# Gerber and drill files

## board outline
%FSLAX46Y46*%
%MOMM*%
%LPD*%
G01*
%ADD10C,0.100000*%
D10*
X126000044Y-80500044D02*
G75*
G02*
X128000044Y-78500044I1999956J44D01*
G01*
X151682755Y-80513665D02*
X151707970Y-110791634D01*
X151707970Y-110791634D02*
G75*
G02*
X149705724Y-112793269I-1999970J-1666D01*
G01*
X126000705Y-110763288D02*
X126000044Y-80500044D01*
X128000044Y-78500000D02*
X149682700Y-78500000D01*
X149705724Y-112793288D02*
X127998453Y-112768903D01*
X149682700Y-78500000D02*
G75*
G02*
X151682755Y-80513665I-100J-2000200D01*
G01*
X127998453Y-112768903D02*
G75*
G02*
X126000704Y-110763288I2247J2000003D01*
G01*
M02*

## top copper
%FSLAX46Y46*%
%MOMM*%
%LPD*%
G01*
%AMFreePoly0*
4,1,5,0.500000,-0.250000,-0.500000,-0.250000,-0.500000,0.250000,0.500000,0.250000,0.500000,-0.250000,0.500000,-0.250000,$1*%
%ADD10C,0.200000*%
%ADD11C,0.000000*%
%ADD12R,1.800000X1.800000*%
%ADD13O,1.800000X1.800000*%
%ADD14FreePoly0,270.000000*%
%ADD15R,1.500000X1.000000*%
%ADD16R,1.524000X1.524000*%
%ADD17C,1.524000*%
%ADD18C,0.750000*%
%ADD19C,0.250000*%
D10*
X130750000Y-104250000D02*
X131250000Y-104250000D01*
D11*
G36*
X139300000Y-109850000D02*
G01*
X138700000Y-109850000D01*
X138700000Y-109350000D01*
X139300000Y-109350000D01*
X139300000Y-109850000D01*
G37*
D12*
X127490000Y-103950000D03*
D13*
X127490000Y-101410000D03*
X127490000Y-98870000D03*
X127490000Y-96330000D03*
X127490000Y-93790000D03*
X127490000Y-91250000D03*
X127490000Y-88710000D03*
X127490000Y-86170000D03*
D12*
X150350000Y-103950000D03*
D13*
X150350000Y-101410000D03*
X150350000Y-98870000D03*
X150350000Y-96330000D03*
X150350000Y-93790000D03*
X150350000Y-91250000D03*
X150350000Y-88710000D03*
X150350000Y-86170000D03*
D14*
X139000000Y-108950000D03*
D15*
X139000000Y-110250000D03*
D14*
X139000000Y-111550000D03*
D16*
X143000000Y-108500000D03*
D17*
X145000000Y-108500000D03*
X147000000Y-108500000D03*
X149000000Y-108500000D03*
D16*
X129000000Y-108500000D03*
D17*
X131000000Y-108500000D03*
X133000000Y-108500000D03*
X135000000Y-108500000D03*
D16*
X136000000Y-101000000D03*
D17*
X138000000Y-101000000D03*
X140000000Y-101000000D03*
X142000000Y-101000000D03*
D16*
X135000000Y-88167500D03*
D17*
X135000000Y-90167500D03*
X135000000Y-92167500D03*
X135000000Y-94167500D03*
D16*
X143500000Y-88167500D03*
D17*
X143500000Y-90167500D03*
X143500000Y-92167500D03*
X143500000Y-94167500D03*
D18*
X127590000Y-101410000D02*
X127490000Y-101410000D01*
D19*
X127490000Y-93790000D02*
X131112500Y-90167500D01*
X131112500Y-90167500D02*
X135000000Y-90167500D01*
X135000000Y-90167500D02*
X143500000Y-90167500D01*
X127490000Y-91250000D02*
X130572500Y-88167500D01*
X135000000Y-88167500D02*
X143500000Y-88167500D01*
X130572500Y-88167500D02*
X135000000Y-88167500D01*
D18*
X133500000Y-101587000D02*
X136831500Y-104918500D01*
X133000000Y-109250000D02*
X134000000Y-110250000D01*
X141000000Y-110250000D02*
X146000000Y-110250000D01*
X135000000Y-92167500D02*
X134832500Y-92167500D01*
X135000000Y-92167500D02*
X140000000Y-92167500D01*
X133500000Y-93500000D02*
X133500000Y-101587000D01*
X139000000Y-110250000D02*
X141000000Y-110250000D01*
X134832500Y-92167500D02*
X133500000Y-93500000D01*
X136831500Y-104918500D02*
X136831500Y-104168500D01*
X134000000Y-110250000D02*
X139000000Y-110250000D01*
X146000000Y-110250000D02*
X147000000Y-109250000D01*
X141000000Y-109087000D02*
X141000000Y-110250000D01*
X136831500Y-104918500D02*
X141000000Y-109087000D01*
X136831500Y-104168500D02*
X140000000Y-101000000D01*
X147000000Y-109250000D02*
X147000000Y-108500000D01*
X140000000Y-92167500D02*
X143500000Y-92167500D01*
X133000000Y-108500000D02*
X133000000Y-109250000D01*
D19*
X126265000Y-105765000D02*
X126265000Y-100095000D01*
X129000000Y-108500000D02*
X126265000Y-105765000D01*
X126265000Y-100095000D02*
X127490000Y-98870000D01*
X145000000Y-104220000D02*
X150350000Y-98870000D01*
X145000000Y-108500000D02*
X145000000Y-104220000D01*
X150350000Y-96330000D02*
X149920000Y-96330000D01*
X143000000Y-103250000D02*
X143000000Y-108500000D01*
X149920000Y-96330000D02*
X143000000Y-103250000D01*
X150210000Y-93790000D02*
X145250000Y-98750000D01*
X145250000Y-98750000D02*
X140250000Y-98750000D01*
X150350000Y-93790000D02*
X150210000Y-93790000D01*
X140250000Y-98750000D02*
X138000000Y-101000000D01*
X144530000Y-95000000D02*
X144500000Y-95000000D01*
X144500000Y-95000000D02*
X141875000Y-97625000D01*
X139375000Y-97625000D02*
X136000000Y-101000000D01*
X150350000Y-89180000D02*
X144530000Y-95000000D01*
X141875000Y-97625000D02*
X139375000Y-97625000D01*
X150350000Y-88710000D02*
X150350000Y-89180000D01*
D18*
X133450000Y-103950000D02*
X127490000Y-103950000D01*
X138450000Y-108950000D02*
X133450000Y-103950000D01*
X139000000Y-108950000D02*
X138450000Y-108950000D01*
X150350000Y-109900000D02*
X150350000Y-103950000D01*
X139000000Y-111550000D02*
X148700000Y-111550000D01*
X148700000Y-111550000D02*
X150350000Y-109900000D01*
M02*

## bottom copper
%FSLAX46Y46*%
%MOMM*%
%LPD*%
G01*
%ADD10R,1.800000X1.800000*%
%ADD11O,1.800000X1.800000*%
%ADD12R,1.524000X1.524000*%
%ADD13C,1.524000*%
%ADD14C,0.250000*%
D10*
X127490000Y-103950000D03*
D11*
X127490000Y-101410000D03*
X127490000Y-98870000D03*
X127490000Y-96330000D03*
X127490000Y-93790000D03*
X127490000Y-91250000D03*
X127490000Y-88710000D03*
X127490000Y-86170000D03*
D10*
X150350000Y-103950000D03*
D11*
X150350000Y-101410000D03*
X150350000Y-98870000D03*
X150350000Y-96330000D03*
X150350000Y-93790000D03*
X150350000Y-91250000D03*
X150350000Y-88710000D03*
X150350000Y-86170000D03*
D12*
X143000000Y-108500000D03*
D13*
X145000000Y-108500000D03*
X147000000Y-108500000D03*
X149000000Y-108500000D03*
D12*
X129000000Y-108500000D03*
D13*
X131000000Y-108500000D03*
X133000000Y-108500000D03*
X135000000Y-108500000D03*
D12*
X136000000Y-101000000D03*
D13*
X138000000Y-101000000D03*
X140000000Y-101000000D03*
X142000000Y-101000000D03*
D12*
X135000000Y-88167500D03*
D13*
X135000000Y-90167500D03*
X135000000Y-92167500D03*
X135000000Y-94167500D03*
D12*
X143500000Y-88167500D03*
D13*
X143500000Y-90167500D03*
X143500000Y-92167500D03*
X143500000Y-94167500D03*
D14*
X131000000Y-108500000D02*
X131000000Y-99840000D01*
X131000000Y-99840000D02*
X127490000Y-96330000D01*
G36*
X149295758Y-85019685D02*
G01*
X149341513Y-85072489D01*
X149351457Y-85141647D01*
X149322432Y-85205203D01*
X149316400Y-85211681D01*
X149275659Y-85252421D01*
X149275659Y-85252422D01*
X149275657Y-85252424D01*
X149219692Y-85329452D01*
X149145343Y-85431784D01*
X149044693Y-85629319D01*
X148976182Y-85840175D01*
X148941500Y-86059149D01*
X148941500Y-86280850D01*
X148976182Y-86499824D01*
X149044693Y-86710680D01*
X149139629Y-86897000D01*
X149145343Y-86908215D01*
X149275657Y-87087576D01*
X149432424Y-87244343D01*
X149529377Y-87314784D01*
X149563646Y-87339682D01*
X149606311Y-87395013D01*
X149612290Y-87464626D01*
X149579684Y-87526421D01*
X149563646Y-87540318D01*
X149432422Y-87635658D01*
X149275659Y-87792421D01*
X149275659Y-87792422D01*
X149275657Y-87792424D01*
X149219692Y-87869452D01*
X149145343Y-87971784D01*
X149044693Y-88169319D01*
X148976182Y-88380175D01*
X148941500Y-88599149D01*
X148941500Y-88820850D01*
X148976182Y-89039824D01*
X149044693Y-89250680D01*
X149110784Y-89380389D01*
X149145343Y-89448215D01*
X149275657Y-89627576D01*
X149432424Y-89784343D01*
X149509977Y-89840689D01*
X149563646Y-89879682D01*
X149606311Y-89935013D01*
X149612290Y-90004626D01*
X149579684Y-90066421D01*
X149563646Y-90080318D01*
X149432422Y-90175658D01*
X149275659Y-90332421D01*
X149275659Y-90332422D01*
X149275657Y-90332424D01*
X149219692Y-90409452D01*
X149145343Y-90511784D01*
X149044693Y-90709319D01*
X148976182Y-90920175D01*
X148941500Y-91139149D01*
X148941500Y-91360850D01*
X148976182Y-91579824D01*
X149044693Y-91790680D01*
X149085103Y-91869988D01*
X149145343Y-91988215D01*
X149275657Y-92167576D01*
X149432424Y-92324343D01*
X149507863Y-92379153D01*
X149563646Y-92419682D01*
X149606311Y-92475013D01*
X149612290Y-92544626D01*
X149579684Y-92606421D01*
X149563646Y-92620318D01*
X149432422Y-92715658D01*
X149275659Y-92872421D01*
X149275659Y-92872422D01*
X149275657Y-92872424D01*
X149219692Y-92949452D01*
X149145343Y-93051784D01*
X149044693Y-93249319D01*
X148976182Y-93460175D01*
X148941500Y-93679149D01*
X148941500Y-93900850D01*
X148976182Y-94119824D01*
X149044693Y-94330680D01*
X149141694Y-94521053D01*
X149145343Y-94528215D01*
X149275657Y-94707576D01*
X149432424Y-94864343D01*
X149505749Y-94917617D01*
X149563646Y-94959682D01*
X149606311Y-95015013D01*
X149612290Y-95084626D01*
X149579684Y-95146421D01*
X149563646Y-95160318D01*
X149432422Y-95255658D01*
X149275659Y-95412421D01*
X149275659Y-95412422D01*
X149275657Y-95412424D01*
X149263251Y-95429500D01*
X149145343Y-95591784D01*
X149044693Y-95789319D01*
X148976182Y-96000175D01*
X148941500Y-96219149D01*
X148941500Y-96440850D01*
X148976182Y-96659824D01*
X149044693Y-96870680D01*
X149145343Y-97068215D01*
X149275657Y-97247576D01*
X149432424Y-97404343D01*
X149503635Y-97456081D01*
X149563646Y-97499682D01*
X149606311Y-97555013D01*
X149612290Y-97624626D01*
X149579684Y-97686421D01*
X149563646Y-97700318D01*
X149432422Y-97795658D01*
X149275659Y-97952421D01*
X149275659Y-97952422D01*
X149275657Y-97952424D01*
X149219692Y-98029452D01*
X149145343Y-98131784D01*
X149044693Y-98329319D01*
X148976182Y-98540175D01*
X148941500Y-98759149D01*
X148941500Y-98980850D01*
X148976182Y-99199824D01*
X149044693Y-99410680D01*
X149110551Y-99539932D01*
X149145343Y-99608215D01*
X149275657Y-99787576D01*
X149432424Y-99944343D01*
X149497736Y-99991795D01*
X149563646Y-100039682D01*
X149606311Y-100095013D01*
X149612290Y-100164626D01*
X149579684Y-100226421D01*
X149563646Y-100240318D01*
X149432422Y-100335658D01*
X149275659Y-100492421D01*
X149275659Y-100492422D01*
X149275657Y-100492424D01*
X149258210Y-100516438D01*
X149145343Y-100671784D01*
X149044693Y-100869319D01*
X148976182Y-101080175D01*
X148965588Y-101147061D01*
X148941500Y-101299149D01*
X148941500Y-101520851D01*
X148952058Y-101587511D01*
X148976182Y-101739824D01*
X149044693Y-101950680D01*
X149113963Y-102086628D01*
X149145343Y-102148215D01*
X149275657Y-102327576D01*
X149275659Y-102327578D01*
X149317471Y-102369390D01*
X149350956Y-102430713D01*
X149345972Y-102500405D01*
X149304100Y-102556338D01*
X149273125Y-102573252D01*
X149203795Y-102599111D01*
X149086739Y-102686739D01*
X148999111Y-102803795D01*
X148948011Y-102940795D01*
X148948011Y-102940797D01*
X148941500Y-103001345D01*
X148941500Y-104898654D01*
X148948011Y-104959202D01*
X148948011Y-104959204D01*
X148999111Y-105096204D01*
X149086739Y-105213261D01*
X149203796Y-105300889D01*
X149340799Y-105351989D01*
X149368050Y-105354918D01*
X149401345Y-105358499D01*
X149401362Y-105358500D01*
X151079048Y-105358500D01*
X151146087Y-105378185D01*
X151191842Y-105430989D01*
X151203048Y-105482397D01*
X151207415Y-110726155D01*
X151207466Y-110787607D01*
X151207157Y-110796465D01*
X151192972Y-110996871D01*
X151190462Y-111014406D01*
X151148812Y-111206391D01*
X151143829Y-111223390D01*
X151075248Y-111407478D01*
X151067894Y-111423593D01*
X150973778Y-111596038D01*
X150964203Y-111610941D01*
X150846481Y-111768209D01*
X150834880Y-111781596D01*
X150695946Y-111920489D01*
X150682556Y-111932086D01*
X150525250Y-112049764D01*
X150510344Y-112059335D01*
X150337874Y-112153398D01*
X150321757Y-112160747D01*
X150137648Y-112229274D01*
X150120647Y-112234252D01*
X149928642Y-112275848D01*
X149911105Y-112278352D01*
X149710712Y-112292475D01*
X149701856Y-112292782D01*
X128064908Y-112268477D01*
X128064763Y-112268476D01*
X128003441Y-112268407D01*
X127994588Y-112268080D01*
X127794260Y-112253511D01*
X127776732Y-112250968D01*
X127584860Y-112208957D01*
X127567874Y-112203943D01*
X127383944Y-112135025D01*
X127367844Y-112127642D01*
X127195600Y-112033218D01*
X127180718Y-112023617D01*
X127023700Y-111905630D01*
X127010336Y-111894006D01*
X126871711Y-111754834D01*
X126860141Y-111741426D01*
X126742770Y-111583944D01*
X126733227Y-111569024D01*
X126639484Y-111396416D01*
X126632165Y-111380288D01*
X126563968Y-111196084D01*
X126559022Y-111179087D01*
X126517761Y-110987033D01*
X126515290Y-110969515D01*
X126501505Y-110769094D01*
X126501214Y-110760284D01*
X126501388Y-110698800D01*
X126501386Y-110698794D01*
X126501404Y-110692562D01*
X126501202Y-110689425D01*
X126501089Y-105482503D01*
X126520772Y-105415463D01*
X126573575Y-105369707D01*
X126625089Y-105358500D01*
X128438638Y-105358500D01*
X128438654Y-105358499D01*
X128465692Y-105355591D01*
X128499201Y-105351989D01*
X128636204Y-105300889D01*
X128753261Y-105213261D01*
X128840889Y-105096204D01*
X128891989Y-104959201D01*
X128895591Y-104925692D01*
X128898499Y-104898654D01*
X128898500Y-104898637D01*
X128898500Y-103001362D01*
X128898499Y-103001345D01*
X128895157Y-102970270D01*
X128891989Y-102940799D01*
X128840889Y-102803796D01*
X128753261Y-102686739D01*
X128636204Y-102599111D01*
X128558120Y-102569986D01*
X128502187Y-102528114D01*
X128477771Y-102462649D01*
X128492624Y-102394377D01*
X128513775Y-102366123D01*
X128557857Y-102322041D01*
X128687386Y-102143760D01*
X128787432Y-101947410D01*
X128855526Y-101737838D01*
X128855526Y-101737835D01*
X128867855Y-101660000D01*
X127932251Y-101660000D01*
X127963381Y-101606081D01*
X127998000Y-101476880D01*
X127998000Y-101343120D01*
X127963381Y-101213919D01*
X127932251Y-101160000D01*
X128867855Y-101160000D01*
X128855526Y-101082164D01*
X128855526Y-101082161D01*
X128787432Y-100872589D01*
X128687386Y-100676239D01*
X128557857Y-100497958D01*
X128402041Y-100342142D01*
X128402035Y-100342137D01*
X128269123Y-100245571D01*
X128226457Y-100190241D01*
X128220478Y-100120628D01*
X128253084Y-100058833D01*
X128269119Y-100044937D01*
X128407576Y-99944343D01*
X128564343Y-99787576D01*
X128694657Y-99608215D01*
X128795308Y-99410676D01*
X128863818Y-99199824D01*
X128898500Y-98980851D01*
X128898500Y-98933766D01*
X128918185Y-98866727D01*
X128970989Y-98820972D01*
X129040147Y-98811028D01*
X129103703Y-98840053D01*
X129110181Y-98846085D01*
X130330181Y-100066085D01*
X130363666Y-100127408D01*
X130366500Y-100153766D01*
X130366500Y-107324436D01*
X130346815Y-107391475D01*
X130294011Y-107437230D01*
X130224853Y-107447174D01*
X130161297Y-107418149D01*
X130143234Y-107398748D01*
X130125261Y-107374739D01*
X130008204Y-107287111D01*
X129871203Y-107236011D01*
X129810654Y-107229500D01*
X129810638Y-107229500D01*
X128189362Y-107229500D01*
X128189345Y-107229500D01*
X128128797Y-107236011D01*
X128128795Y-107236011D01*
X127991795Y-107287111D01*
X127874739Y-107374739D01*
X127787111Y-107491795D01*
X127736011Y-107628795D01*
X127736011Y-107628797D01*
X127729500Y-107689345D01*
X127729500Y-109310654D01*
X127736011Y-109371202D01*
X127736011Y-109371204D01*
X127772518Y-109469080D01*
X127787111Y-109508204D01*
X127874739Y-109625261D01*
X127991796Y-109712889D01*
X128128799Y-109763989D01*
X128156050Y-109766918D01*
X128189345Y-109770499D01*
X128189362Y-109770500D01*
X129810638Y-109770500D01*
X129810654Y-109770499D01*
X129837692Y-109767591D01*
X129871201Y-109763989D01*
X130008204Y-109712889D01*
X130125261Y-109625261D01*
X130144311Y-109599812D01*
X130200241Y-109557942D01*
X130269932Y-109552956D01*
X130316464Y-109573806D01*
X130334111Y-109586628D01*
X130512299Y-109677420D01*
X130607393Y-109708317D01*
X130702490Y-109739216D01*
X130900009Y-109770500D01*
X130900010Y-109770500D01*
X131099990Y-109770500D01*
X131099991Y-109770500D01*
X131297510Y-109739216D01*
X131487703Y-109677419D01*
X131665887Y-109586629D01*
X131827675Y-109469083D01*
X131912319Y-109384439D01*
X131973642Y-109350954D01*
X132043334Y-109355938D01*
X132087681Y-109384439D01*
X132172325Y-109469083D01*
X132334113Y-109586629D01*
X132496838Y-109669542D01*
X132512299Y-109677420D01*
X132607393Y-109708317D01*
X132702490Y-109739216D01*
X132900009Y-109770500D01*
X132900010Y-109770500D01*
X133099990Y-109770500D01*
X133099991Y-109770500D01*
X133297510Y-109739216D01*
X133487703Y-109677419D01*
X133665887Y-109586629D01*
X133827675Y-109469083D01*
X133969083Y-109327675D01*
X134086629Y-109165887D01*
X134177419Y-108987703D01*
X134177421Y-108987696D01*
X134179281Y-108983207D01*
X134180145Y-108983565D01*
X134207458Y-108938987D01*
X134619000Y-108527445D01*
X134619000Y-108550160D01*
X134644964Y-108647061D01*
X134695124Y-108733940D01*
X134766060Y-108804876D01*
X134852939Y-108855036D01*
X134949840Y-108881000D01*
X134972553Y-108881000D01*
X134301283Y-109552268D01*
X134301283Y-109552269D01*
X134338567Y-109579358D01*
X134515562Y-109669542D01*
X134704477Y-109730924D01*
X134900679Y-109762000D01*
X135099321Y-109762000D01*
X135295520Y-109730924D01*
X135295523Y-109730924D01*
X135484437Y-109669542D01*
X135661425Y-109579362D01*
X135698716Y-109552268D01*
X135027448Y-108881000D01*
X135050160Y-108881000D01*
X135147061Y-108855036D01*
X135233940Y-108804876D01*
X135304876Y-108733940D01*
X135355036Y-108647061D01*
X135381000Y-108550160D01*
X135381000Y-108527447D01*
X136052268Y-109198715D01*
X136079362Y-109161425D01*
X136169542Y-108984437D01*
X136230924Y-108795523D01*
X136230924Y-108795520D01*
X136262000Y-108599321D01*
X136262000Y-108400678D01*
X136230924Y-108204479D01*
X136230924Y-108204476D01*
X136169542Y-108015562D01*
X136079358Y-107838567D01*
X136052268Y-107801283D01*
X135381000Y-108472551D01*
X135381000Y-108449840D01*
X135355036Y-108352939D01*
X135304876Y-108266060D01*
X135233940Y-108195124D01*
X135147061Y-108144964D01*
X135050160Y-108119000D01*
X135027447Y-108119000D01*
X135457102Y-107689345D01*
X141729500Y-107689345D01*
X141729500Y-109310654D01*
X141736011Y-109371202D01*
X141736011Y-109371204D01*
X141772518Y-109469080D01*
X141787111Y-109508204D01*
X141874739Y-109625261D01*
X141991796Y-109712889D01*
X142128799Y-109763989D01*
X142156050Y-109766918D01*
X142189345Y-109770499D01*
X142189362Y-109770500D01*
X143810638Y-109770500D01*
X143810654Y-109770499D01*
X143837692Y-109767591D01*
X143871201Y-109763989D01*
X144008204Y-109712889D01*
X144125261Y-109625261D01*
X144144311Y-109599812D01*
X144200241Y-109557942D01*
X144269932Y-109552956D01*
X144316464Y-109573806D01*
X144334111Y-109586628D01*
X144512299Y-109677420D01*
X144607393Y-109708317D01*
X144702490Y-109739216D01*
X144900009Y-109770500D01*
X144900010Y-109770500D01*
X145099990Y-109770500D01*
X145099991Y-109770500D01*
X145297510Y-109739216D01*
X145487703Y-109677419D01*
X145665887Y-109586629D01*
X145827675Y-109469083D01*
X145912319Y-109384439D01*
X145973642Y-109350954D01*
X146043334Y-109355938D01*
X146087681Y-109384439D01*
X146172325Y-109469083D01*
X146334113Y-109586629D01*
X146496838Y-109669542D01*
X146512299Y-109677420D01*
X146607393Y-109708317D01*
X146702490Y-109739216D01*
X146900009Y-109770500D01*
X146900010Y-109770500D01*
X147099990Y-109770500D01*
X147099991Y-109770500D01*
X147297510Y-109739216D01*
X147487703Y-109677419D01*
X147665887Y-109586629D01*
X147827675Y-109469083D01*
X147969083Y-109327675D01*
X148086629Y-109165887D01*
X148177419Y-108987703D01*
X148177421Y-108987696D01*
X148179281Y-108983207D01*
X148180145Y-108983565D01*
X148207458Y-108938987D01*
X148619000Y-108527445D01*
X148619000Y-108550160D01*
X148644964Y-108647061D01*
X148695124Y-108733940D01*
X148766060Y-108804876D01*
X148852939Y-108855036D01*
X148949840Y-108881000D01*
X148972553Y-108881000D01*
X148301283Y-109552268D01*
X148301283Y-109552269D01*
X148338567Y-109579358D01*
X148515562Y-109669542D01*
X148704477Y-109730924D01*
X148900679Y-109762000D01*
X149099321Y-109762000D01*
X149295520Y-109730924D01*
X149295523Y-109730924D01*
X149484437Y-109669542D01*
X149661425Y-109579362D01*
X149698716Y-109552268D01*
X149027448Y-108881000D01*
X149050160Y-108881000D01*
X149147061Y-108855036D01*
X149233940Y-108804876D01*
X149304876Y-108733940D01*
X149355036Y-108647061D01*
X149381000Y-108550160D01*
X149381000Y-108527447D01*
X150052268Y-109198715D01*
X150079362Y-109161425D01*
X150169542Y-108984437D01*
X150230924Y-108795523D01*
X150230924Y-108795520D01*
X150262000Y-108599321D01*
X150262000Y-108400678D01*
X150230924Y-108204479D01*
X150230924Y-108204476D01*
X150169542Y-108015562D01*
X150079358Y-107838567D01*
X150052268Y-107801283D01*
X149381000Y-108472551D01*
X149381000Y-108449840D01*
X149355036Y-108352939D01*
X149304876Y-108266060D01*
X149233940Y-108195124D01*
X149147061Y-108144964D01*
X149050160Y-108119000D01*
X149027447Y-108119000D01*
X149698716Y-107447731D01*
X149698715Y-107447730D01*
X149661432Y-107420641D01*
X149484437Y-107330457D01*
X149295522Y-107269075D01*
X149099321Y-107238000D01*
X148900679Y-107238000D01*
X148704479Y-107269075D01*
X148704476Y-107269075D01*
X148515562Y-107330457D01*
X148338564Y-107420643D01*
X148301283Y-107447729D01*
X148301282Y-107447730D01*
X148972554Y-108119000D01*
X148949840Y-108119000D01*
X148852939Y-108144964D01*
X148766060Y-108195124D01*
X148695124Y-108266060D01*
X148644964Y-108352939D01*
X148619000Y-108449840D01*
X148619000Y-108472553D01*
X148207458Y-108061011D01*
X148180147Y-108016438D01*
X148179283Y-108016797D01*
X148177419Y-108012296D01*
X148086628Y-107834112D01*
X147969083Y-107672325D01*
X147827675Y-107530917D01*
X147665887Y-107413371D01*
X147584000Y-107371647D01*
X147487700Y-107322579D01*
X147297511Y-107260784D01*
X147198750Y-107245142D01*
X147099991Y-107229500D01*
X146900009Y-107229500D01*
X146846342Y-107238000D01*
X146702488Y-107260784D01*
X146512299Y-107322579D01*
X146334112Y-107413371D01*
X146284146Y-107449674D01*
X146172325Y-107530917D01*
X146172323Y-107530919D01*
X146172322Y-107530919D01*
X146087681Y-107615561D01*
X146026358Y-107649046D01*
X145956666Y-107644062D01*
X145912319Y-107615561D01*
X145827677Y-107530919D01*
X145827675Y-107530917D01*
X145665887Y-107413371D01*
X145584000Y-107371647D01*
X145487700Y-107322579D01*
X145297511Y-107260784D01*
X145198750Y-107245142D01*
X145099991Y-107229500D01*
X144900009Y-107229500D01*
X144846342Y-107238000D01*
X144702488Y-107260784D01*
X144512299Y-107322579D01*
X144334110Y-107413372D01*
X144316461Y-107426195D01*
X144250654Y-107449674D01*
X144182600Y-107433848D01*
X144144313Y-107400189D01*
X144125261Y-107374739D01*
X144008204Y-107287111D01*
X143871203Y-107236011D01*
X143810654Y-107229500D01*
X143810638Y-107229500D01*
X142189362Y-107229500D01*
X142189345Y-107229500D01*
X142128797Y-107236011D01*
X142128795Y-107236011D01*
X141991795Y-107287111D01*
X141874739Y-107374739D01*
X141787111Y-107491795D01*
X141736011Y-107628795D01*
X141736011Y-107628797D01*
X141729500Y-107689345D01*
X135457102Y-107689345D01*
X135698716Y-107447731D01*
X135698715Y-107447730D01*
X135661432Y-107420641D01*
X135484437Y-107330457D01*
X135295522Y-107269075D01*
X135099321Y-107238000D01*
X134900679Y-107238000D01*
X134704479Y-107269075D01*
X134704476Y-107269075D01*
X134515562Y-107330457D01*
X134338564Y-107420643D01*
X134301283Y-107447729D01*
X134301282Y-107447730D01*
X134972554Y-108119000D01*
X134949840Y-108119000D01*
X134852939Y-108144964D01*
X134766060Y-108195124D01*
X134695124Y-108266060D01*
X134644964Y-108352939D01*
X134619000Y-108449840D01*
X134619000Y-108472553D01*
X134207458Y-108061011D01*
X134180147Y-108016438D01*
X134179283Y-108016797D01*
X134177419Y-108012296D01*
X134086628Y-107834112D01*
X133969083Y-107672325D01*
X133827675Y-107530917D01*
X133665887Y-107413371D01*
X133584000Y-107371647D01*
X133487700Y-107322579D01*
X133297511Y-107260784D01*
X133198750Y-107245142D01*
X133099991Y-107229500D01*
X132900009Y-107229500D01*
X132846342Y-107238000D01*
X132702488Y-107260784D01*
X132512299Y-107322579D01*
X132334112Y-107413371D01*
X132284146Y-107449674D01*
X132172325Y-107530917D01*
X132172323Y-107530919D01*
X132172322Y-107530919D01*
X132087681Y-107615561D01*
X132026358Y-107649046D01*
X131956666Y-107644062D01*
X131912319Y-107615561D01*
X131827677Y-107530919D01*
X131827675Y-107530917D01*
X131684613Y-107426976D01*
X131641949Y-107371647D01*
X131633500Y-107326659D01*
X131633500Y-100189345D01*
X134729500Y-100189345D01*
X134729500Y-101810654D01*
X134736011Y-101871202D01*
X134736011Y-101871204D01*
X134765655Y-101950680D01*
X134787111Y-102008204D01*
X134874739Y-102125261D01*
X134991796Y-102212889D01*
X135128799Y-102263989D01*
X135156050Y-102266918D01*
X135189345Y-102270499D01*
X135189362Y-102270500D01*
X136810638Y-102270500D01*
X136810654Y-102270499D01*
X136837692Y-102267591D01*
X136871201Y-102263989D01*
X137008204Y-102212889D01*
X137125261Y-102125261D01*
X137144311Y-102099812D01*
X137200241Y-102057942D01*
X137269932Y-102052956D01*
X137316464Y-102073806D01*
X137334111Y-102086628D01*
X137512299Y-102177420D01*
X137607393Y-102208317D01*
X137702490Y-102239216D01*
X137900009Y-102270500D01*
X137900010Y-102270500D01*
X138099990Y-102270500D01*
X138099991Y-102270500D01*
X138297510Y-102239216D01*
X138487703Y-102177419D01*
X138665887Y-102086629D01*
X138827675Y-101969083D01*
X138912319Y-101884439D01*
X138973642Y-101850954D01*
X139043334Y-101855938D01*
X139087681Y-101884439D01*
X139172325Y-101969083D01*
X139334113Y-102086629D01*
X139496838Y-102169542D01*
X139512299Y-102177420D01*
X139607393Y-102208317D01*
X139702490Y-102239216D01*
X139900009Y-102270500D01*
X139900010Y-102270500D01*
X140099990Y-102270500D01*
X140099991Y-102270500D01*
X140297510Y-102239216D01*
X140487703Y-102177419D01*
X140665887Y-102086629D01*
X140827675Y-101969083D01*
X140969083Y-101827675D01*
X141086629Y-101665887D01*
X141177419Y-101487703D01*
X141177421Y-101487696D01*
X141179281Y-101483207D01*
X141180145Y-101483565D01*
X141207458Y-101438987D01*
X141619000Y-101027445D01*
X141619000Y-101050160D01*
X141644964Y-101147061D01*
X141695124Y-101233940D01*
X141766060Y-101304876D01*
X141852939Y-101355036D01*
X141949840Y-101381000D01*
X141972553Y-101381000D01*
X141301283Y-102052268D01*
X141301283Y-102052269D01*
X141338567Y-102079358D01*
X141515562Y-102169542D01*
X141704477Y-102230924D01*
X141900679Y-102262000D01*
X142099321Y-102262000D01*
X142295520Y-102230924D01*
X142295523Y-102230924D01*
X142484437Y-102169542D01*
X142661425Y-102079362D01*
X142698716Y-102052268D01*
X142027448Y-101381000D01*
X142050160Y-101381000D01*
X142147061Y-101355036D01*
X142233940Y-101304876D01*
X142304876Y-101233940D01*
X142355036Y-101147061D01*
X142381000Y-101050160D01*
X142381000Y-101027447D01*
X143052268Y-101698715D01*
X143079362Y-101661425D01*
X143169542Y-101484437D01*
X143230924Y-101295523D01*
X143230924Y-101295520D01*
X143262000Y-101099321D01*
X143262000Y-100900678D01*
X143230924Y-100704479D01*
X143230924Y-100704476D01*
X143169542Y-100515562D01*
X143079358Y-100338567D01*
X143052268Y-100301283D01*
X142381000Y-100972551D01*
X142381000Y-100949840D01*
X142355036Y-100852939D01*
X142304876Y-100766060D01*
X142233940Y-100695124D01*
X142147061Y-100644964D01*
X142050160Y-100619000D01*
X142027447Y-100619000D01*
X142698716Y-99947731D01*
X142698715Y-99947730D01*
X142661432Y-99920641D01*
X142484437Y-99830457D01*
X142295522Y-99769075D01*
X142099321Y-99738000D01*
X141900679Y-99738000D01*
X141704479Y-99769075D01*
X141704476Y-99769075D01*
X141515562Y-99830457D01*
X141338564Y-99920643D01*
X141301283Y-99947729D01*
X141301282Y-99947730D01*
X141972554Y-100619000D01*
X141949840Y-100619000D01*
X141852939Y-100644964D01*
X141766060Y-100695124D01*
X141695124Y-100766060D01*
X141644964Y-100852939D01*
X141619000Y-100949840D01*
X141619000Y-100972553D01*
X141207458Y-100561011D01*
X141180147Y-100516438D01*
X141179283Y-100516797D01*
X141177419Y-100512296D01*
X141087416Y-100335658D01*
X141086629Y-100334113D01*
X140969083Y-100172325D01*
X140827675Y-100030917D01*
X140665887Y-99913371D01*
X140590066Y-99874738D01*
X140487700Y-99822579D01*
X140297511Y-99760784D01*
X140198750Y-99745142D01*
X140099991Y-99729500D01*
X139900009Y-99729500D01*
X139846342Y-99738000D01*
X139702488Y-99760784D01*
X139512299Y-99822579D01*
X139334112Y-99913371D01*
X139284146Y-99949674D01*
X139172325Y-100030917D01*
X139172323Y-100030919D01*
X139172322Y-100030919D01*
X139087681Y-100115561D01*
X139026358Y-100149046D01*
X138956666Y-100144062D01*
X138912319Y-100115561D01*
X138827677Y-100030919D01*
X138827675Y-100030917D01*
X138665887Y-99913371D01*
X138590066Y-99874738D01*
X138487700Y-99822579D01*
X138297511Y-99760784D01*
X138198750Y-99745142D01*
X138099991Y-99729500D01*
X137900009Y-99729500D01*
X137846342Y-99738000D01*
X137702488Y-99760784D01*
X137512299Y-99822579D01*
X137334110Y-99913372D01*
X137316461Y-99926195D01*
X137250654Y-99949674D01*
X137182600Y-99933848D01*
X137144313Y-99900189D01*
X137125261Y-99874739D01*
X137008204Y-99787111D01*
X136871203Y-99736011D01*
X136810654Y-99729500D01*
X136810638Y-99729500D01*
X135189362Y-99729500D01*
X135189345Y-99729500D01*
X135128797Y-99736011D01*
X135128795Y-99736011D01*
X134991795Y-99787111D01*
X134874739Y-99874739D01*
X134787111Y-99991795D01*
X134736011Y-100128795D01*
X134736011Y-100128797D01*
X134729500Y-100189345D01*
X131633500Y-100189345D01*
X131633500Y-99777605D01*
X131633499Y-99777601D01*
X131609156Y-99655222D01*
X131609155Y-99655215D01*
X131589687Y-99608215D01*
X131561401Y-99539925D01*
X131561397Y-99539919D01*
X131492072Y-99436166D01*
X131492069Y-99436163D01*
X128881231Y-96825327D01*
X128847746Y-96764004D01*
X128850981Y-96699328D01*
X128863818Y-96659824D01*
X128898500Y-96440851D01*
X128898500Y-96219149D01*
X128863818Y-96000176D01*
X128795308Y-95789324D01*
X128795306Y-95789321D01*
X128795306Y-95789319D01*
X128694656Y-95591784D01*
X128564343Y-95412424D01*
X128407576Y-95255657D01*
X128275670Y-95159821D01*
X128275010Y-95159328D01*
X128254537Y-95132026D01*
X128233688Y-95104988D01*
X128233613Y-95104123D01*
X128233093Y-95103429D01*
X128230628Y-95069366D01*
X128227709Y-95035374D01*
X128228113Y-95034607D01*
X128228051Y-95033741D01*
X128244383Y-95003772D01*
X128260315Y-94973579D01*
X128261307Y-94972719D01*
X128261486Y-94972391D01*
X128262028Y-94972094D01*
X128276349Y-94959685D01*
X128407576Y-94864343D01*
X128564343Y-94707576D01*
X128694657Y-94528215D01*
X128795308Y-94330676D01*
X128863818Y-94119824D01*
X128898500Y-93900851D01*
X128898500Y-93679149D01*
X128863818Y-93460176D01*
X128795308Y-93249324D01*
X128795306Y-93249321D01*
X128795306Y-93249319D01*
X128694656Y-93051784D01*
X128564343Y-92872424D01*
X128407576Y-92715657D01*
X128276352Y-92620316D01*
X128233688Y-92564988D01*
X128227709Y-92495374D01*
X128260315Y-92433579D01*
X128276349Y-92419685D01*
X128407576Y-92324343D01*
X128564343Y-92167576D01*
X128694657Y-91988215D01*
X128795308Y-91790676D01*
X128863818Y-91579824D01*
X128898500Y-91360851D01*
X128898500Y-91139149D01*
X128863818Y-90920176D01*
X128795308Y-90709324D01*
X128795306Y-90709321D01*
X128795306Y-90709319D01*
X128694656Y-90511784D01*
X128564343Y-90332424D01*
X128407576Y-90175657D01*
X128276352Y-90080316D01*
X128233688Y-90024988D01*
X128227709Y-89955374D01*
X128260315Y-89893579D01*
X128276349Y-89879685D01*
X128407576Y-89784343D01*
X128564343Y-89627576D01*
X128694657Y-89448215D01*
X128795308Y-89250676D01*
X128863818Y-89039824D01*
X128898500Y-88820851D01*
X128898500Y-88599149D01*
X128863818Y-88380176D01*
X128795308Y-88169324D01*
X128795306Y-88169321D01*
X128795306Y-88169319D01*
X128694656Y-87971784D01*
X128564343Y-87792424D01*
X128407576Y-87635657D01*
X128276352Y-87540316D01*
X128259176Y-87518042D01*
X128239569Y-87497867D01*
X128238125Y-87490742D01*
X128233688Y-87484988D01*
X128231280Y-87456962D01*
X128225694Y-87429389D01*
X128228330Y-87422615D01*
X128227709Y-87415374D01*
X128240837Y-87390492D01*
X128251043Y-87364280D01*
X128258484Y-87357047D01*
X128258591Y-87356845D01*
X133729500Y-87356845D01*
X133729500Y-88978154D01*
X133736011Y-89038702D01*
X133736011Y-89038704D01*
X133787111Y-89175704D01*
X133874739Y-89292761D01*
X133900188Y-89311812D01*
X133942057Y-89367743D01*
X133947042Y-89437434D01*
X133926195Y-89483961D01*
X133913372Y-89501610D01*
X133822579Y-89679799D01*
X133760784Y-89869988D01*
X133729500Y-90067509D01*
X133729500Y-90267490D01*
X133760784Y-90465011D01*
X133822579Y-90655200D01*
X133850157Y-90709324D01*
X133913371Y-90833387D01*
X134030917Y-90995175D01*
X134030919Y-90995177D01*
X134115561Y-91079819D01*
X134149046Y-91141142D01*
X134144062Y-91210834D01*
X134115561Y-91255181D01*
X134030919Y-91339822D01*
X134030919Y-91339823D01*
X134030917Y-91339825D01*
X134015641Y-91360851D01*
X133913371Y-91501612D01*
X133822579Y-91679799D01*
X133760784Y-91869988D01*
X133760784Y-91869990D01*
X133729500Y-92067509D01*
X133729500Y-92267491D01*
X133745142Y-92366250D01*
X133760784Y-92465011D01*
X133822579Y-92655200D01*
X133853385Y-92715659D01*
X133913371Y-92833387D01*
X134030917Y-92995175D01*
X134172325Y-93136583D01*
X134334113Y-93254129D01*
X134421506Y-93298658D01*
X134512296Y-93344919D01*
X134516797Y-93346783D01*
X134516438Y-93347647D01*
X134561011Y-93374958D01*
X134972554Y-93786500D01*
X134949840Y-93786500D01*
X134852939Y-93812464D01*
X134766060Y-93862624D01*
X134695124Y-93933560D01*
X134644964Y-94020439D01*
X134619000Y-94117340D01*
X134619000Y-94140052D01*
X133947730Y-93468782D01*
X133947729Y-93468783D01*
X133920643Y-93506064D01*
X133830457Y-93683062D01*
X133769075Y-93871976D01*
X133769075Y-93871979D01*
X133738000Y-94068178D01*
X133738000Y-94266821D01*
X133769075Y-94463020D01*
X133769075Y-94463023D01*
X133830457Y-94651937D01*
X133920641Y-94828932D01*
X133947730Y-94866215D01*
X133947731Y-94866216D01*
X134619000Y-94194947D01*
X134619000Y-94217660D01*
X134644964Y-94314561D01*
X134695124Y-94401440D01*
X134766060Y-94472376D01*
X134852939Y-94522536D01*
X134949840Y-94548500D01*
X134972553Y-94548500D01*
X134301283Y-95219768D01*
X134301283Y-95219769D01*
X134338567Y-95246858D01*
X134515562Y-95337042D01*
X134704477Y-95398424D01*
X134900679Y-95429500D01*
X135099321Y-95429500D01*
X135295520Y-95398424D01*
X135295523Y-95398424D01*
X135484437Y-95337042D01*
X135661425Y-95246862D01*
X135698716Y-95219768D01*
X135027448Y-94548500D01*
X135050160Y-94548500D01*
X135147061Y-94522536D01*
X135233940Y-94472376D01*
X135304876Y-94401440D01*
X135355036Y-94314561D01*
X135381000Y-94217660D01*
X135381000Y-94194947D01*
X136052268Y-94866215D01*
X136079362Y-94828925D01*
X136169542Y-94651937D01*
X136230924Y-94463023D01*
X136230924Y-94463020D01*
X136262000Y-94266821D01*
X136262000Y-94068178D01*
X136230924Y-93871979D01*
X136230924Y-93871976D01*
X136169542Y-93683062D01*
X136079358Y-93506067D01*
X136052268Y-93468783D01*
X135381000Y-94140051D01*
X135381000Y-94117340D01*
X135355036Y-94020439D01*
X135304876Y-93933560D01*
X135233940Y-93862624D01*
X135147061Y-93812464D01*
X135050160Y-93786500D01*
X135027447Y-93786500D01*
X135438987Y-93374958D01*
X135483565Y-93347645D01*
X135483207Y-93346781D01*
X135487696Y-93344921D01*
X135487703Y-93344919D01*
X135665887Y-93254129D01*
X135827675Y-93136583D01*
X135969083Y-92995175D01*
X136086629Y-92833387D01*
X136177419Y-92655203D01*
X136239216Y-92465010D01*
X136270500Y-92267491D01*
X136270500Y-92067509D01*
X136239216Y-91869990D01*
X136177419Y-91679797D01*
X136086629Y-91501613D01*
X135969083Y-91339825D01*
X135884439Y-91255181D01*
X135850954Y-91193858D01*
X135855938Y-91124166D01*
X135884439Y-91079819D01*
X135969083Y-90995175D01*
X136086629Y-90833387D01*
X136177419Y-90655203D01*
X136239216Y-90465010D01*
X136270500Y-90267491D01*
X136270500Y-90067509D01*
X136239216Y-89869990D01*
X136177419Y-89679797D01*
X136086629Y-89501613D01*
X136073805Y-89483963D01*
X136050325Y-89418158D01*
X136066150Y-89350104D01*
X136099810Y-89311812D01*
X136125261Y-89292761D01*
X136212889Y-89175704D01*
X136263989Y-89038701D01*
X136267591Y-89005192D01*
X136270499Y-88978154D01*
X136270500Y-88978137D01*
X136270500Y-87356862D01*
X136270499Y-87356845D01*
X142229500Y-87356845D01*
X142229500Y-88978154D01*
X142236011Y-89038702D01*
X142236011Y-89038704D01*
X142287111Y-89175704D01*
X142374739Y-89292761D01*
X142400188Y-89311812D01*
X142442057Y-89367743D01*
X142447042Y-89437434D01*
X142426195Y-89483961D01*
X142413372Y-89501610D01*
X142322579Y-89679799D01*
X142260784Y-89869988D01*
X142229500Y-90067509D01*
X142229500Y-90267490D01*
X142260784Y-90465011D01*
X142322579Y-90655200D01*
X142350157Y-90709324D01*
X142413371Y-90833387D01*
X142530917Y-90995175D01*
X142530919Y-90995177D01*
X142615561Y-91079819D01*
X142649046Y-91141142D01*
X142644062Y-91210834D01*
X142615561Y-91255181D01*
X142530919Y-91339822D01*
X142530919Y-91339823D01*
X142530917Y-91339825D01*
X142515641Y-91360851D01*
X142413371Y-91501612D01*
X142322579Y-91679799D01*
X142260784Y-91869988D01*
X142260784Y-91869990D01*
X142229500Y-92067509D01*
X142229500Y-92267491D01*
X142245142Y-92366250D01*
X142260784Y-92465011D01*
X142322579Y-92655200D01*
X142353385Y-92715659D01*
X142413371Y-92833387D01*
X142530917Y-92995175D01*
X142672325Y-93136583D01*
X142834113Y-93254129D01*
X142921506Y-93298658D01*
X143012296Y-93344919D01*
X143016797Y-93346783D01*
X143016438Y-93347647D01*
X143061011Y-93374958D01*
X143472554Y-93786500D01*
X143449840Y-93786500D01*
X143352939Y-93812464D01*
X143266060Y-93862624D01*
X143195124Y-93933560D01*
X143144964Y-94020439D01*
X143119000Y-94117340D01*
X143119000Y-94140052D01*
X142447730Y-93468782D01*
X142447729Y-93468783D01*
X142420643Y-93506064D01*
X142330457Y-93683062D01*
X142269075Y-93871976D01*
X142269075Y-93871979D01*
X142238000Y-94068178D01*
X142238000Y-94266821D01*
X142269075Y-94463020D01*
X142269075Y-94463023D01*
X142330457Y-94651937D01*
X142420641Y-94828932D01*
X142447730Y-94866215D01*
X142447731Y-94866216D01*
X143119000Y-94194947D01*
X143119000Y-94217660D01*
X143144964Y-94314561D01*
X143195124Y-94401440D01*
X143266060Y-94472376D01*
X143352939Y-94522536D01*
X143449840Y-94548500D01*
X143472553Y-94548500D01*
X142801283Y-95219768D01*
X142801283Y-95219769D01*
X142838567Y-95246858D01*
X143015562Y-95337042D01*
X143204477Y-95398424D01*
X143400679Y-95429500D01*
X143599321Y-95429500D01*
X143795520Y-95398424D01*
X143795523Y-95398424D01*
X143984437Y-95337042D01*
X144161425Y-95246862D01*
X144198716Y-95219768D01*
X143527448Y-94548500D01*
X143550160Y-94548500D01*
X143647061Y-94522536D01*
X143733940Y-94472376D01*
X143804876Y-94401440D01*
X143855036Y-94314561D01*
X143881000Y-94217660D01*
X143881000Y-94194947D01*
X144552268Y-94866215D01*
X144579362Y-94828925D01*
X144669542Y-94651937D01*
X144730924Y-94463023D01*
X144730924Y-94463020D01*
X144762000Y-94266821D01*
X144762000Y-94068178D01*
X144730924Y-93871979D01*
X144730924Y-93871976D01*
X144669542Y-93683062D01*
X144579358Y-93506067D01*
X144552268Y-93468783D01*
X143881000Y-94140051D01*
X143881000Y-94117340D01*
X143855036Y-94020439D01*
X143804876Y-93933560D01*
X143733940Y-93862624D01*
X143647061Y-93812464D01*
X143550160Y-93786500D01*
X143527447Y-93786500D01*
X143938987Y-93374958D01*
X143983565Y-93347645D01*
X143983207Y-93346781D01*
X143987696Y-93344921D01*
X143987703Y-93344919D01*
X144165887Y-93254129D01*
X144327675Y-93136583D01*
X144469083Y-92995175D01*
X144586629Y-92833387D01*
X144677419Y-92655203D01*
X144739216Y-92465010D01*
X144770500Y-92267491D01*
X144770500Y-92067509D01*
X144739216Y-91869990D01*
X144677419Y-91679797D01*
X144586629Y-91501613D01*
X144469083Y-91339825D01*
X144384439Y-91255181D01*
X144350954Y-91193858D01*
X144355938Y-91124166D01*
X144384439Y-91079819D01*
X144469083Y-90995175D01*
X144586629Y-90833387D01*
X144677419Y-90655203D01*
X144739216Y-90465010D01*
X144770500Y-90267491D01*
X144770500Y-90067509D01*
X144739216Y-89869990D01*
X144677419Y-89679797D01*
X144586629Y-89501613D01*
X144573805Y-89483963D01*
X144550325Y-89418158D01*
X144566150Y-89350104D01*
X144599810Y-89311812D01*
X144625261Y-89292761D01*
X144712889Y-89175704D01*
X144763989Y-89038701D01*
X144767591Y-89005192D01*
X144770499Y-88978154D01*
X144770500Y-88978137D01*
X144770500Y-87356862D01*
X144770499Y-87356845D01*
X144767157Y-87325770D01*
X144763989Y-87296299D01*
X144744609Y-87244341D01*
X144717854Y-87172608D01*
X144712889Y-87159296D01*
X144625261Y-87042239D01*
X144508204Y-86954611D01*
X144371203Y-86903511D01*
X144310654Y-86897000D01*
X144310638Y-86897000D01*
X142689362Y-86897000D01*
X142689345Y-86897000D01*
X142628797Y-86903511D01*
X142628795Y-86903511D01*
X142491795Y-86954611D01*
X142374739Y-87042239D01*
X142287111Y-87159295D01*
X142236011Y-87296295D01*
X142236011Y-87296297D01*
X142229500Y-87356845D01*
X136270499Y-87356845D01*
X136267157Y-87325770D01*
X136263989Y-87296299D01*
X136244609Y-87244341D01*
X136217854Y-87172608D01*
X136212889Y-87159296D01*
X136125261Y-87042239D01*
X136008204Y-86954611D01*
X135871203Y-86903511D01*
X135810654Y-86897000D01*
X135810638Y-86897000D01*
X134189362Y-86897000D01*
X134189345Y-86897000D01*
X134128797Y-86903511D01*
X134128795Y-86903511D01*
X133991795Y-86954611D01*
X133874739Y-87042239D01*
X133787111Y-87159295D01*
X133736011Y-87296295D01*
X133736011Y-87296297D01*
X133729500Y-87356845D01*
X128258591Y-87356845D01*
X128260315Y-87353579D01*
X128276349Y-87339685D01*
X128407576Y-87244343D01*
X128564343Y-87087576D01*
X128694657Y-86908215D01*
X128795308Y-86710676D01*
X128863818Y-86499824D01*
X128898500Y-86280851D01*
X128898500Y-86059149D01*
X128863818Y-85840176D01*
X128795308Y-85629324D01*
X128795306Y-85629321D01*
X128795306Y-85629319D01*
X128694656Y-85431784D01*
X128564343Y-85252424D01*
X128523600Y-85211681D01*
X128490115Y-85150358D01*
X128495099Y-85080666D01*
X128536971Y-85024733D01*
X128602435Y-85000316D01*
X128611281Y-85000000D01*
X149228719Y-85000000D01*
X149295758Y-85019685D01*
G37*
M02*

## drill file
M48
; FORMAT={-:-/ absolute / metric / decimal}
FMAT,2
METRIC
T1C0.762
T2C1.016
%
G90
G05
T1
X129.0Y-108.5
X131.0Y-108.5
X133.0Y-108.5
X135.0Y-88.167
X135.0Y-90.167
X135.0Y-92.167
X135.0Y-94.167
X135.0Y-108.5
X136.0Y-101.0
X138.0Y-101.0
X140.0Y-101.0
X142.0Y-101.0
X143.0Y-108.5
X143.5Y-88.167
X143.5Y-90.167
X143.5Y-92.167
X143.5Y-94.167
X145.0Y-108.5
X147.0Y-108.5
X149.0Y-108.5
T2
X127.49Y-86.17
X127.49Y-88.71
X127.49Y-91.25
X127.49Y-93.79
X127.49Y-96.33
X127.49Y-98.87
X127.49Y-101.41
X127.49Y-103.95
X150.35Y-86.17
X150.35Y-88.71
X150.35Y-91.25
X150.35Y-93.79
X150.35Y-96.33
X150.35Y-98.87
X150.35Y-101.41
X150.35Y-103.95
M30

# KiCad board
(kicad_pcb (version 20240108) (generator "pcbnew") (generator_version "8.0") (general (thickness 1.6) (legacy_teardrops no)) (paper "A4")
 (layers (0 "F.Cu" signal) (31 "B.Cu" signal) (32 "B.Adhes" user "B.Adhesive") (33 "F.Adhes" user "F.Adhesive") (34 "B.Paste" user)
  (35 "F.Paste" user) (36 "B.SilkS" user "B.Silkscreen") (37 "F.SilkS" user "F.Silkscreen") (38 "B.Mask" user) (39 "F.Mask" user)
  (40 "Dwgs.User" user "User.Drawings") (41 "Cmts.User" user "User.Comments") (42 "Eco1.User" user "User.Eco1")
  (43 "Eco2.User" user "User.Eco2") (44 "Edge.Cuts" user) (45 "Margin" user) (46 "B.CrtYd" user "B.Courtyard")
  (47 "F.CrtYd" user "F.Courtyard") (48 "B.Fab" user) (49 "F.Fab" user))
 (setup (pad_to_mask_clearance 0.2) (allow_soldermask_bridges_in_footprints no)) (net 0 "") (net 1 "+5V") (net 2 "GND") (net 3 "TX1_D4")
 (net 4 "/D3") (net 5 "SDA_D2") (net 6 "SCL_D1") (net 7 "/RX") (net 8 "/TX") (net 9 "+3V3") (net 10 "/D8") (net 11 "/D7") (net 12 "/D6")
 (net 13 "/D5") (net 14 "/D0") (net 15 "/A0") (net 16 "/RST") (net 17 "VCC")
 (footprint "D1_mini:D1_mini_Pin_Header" (layer "F.Cu") (at 127.49 103.95 180)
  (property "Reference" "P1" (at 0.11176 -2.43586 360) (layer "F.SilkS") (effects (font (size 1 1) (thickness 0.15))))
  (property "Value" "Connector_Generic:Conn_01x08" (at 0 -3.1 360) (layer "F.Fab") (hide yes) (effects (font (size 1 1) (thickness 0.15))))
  (pad "1" thru_hole rect (at 0 0 180) (size 1.8 1.8) (drill 1.016) (layers "*.Cu" "*.Mask" "F.SilkS") (remove_unused_layers no)
   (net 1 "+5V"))
  (pad "2" thru_hole oval (at 0 2.54 180) (size 1.8 1.8) (drill 1.016) (layers "*.Cu" "*.Mask" "F.SilkS") (remove_unused_layers no)
   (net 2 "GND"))
  (pad "3" thru_hole oval (at 0 5.08 180) (size 1.8 1.8) (drill 1.016) (layers "*.Cu" "*.Mask" "F.SilkS") (remove_unused_layers no)
   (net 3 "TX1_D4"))
  (pad "4" thru_hole oval (at 0 7.62 180) (size 1.8 1.8) (drill 1.016) (layers "*.Cu" "*.Mask" "F.SilkS") (remove_unused_layers no)
   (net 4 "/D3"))
  (pad "5" thru_hole oval (at 0 10.16 180) (size 1.8 1.8) (drill 1.016) (layers "*.Cu" "*.Mask" "F.SilkS") (remove_unused_layers no)
   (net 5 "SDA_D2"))
  (pad "6" thru_hole oval (at 0 12.7 180) (size 1.8 1.8) (drill 1.016) (layers "*.Cu" "*.Mask" "F.SilkS") (remove_unused_layers no)
   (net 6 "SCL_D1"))
  (pad "7" thru_hole oval (at 0 15.24 180) (size 1.8 1.8) (drill 1.016) (layers "*.Cu" "*.Mask" "F.SilkS") (remove_unused_layers no)
   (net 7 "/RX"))
  (pad "8" thru_hole oval (at 0 17.78 180) (size 1.8 1.8) (drill 1.016) (layers "*.Cu" "*.Mask" "F.SilkS") (remove_unused_layers no)
   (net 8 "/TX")))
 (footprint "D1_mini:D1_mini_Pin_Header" (layer "F.Cu") (at 150.35 103.95 180)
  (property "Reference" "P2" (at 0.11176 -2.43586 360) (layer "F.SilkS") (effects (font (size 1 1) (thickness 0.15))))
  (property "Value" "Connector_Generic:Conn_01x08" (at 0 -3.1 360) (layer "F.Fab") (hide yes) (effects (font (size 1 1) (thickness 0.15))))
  (pad "1" thru_hole rect (at 0 0 180) (size 1.8 1.8) (drill 1.016) (layers "*.Cu" "*.Mask" "F.SilkS") (remove_unused_layers no)
   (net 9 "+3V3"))
  (pad "2" thru_hole oval (at 0 2.54 180) (size 1.8 1.8) (drill 1.016) (layers "*.Cu" "*.Mask" "F.SilkS") (remove_unused_layers no)
   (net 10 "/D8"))
  (pad "3" thru_hole oval (at 0 5.08 180) (size 1.8 1.8) (drill 1.016) (layers "*.Cu" "*.Mask" "F.SilkS") (remove_unused_layers no)
   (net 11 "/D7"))
  (pad "4" thru_hole oval (at 0 7.62 180) (size 1.8 1.8) (drill 1.016) (layers "*.Cu" "*.Mask" "F.SilkS") (remove_unused_layers no)
   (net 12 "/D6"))
  (pad "5" thru_hole oval (at 0 10.16 180) (size 1.8 1.8) (drill 1.016) (layers "*.Cu" "*.Mask" "F.SilkS") (remove_unused_layers no)
   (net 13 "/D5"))
  (pad "6" thru_hole oval (at 0 12.7 180) (size 1.8 1.8) (drill 1.016) (layers "*.Cu" "*.Mask" "F.SilkS") (remove_unused_layers no)
   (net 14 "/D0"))
  (pad "7" thru_hole oval (at 0 15.24 180) (size 1.8 1.8) (drill 1.016) (layers "*.Cu" "*.Mask" "F.SilkS") (remove_unused_layers no)
   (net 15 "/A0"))
  (pad "8" thru_hole oval (at 0 17.78 180) (size 1.8 1.8) (drill 1.016) (layers "*.Cu" "*.Mask" "F.SilkS") (remove_unused_layers no)
   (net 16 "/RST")))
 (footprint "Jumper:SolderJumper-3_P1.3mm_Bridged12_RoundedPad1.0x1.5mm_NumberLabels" (layer "F.Cu") (at 139 110.25 -90)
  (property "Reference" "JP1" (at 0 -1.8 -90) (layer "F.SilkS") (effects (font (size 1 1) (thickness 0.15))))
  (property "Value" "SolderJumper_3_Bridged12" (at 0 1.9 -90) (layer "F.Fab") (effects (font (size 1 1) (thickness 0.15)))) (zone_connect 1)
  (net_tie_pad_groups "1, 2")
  (fp_poly (pts (xy -0.9 -0.3) (xy -0.4 -0.3) (xy -0.4 0.3) (xy -0.9 0.3)) (stroke (width 0) (type solid)) (fill solid) (layer "F.Cu"))
  (pad "1" smd custom (at -1.3 0 270) (size 1 0.5) (layers "F.Cu" "F.Mask") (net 1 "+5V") (zone_connect 2) (thermal_bridge_angle 45)
   (options (clearance outline) (anchor rect)) (primitives))
  (pad "2" smd rect (at 0 0 270) (size 1 1.5) (layers "F.Cu" "F.Mask") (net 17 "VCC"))
  (pad "3" smd custom (at 1.3 0 270) (size 1 0.5) (layers "F.Cu" "F.Mask") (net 9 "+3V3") (zone_connect 2) (thermal_bridge_angle 45)
   (options (clearance outline) (anchor rect)) (primitives)))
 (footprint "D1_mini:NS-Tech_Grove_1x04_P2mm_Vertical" (layer "B.Cu") (at 143 108.5 -90)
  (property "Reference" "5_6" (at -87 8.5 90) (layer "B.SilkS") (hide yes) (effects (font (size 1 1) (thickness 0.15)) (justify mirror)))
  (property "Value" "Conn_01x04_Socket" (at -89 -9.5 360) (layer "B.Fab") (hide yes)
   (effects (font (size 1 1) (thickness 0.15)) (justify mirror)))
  (pad "1" thru_hole rect (at 0 0 270) (size 1.524 1.524) (drill 0.762) (layers "*.Cu" "*.Mask") (remove_unused_layers no) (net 12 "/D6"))
  (pad "2" thru_hole circle (at 0 -2 270) (size 1.524 1.524) (drill 0.762) (layers "*.Cu" "*.Mask") (remove_unused_layers no) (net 11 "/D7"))
  (pad "3" thru_hole circle (at 0 -4 270) (size 1.524 1.524) (drill 0.762) (layers "*.Cu" "*.Mask") (remove_unused_layers no) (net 17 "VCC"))
  (pad "4" thru_hole circle (at 0 -6 270) (size 1.524 1.524) (drill 0.762) (layers "*.Cu" "*.Mask") (remove_unused_layers no) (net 2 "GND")))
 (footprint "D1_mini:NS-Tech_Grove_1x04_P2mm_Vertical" (layer "B.Cu") (at 129 108.5 -90)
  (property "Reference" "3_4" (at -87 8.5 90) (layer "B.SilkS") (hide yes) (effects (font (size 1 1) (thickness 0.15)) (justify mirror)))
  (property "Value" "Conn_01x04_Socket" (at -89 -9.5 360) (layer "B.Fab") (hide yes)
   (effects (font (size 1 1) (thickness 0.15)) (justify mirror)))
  (pad "1" thru_hole rect (at 0 0 270) (size 1.524 1.524) (drill 0.762) (layers "*.Cu" "*.Mask") (remove_unused_layers no) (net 3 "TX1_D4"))
  (pad "2" thru_hole circle (at 0 -2 270) (size 1.524 1.524) (drill 0.762) (layers "*.Cu" "*.Mask") (remove_unused_layers no) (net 4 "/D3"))
  (pad "3" thru_hole circle (at 0 -4 270) (size 1.524 1.524) (drill 0.762) (layers "*.Cu" "*.Mask") (remove_unused_layers no) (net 17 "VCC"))
  (pad "4" thru_hole circle (at 0 -6 270) (size 1.524 1.524) (drill 0.762) (layers "*.Cu" "*.Mask") (remove_unused_layers no) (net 2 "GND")))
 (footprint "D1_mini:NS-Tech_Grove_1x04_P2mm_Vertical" (layer "B.Cu") (at 136 101 -90)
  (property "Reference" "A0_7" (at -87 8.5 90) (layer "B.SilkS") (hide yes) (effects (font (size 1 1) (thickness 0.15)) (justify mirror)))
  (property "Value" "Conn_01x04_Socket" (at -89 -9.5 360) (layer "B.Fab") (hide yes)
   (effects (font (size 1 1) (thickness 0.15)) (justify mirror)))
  (pad "1" thru_hole rect (at 0 0 270) (size 1.524 1.524) (drill 0.762) (layers "*.Cu" "*.Mask") (remove_unused_layers no) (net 15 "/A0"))
  (pad "2" thru_hole circle (at 0 -2 270) (size 1.524 1.524) (drill 0.762) (layers "*.Cu" "*.Mask") (remove_unused_layers no) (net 13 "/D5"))
  (pad "3" thru_hole circle (at 0 -4 270) (size 1.524 1.524) (drill 0.762) (layers "*.Cu" "*.Mask") (remove_unused_layers no) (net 17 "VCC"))
  (pad "4" thru_hole circle (at 0 -6 270) (size 1.524 1.524) (drill 0.762) (layers "*.Cu" "*.Mask") (remove_unused_layers no) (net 2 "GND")))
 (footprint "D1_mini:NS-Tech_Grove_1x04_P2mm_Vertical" (layer "B.Cu") (at 135 88.1675 180)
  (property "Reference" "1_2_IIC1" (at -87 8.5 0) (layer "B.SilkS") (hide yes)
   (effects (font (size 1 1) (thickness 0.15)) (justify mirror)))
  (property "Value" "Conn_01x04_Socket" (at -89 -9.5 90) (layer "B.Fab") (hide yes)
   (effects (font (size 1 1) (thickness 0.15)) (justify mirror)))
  (pad "1" thru_hole rect (at 0 0 180) (size 1.524 1.524) (drill 0.762) (layers "*.Cu" "*.Mask") (remove_unused_layers no) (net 6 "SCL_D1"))
  (pad "2" thru_hole circle (at 0 -2 180) (size 1.524 1.524) (drill 0.762) (layers "*.Cu" "*.Mask") (remove_unused_layers no)
   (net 5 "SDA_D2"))
  (pad "3" thru_hole circle (at 0 -4 180) (size 1.524 1.524) (drill 0.762) (layers "*.Cu" "*.Mask") (remove_unused_layers no) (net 17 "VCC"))
  (pad "4" thru_hole circle (at 0 -6 180) (size 1.524 1.524) (drill 0.762) (layers "*.Cu" "*.Mask") (remove_unused_layers no) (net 2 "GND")))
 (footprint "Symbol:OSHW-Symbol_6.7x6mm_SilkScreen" (layer "B.Cu") (at 147.9 81.75 180)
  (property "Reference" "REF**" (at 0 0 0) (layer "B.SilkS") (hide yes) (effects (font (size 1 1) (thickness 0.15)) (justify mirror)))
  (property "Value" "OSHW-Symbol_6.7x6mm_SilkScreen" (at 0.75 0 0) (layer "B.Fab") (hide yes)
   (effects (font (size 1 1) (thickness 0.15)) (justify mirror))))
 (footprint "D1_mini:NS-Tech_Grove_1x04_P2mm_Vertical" (layer "B.Cu") (at 143.5 88.1675 180)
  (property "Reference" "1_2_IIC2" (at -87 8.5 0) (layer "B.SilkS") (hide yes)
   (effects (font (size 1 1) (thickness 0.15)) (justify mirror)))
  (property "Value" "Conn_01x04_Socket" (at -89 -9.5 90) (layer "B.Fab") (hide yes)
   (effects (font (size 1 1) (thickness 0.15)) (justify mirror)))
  (pad "1" thru_hole rect (at 0 0 180) (size 1.524 1.524) (drill 0.762) (layers "*.Cu" "*.Mask") (remove_unused_layers no) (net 6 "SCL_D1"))
  (pad "2" thru_hole circle (at 0 -2 180) (size 1.524 1.524) (drill 0.762) (layers "*.Cu" "*.Mask") (remove_unused_layers no)
   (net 5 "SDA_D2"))
  (pad "3" thru_hole circle (at 0 -4 180) (size 1.524 1.524) (drill 0.762) (layers "*.Cu" "*.Mask") (remove_unused_layers no) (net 17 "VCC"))
  (pad "4" thru_hole circle (at 0 -6 180) (size 1.524 1.524) (drill 0.762) (layers "*.Cu" "*.Mask") (remove_unused_layers no) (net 2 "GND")))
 (gr_line (start 130.75 104.25) (end 131.25 104.25) (stroke (width 0.2) (type default)) (layer "F.Cu") (net 1))
 (gr_arc (start 126.000044 80.500044) (mid 126.585815 79.085802) (end 128.000044 78.5) (stroke (width 0.1) (type default))
  (layer "Edge.Cuts"))
 (gr_line (start 151.682755 80.513665) (end 151.70797 110.791634) (stroke (width 0.1) (type solid)) (layer "Edge.Cuts"))
 (gr_arc (start 151.70797 110.791634) (mid 151.122062 112.207625) (end 149.705724 112.793288) (stroke (width 0.1) (type default))
  (layer "Edge.Cuts"))
 (gr_line (start 126.000705 110.763288) (end 126.000044 80.500044) (stroke (width 0.1) (type solid)) (layer "Edge.Cuts"))
 (gr_line (start 128.000044 78.5) (end 149.6827 78.5) (stroke (width 0.1) (type solid)) (layer "Edge.Cuts"))
 (gr_line (start 149.705724 112.793288) (end 127.998453 112.768903) (stroke (width 0.1) (type solid)) (layer "Edge.Cuts"))
 (gr_arc (start 149.6827 78.5) (mid 151.09634 79.085213) (end 151.682755 80.513665) (stroke (width 0.1) (type default)) (layer "Edge.Cuts"))
 (gr_arc (start 127.998453 112.768903) (mid 126.585375 112.182007) (end 126.000705 110.763288) (stroke (width 0.1) (type default))
  (layer "Edge.Cuts"))
 (segment (start 127.59 101.41) (end 127.49 101.41) (width 0.75) (layer "F.Cu") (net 2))
 (segment (start 127.49 93.79) (end 131.1125 90.1675) (width 0.25) (layer "F.Cu") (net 5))
 (segment (start 131.1125 90.1675) (end 135 90.1675) (width 0.25) (layer "F.Cu") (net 5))
 (segment (start 135 90.1675) (end 143.5 90.1675) (width 0.25) (layer "F.Cu") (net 5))
 (segment (start 131 108.5) (end 131 99.84) (width 0.25) (layer "B.Cu") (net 4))
 (segment (start 131 99.84) (end 127.49 96.33) (width 0.25) (layer "B.Cu") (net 4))
 (segment (start 127.49 91.25) (end 130.5725 88.1675) (width 0.25) (layer "F.Cu") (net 6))
 (segment (start 135 88.1675) (end 143.5 88.1675) (width 0.25) (layer "F.Cu") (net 6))
 (segment (start 130.5725 88.1675) (end 135 88.1675) (width 0.25) (layer "F.Cu") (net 6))
 (segment (start 133.5 101.587) (end 136.8315 104.9185) (width 0.75) (layer "F.Cu") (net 17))
 (segment (start 133 109.25) (end 134 110.25) (width 0.75) (layer "F.Cu") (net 17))
 (segment (start 141 110.25) (end 146 110.25) (width 0.75) (layer "F.Cu") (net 17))
 (segment (start 135 92.1675) (end 134.8325 92.1675) (width 0.75) (layer "F.Cu") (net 17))
 (segment (start 135 92.1675) (end 140 92.1675) (width 0.75) (layer "F.Cu") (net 17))
 (segment (start 133.5 93.5) (end 133.5 101.587) (width 0.75) (layer "F.Cu") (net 17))
 (segment (start 139 110.25) (end 141 110.25) (width 0.75) (layer "F.Cu") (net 17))
 (segment (start 134.8325 92.1675) (end 133.5 93.5) (width 0.75) (layer "F.Cu") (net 17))
 (segment (start 136.8315 104.9185) (end 136.8315 104.1685) (width 0.75) (layer "F.Cu") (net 17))
 (segment (start 134 110.25) (end 139 110.25) (width 0.75) (layer "F.Cu") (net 17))
 (segment (start 146 110.25) (end 147 109.25) (width 0.75) (layer "F.Cu") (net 17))
 (segment (start 141 109.087) (end 141 110.25) (width 0.75) (layer "F.Cu") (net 17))
 (segment (start 136.8315 104.9185) (end 141 109.087) (width 0.75) (layer "F.Cu") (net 17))
 (segment (start 136.8315 104.1685) (end 140 101) (width 0.75) (layer "F.Cu") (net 17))
 (segment (start 147 109.25) (end 147 108.5) (width 0.75) (layer "F.Cu") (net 17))
 (segment (start 140 92.1675) (end 143.5 92.1675) (width 0.75) (layer "F.Cu") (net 17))
 (segment (start 133 108.5) (end 133 109.25) (width 0.75) (layer "F.Cu") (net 17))
 (segment (start 126.265 105.765) (end 126.265 100.095) (width 0.25) (layer "F.Cu") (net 3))
 (segment (start 129 108.5) (end 126.265 105.765) (width 0.25) (layer "F.Cu") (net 3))
 (segment (start 126.265 100.095) (end 127.49 98.87) (width 0.25) (layer "F.Cu") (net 3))
 (segment (start 145 104.22) (end 150.35 98.87) (width 0.25) (layer "F.Cu") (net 11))
 (segment (start 145 108.5) (end 145 104.22) (width 0.25) (layer "F.Cu") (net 11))
 (segment (start 150.35 96.33) (end 149.92 96.33) (width 0.25) (layer "F.Cu") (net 12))
 (segment (start 143 103.25) (end 143 108.5) (width 0.25) (layer "F.Cu") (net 12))
 (segment (start 149.92 96.33) (end 143 103.25) (width 0.25) (layer "F.Cu") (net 12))
 (segment (start 150.21 93.79) (end 145.25 98.75) (width 0.25) (layer "F.Cu") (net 13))
 (segment (start 145.25 98.75) (end 140.25 98.75) (width 0.25) (layer "F.Cu") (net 13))
 (segment (start 150.35 93.79) (end 150.21 93.79) (width 0.25) (layer "F.Cu") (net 13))
 (segment (start 140.25 98.75) (end 138 101) (width 0.25) (layer "F.Cu") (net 13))
 (segment (start 144.53 95) (end 144.5 95) (width 0.25) (layer "F.Cu") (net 15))
 (segment (start 144.5 95) (end 141.875 97.625) (width 0.25) (layer "F.Cu") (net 15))
 (segment (start 139.375 97.625) (end 136 101) (width 0.25) (layer "F.Cu") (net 15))
 (segment (start 150.35 89.18) (end 144.53 95) (width 0.25) (layer "F.Cu") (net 15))
 (segment (start 141.875 97.625) (end 139.375 97.625) (width 0.25) (layer "F.Cu") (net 15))
 (segment (start 150.35 88.71) (end 150.35 89.18) (width 0.25) (layer "F.Cu") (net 15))
 (segment (start 133.45 103.95) (end 127.49 103.95) (width 0.75) (layer "F.Cu") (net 1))
 (segment (start 138.45 108.95) (end 133.45 103.95) (width 0.75) (layer "F.Cu") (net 1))
 (segment (start 139 108.95) (end 138.45 108.95) (width 0.75) (layer "F.Cu") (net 1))
 (segment (start 150.35 109.9) (end 150.35 103.95) (width 0.75) (layer "F.Cu") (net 9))
 (segment (start 139 111.55) (end 148.7 111.55) (width 0.75) (layer "F.Cu") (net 9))
 (segment (start 148.7 111.55) (end 150.35 109.9) (width 0.75) (layer "F.Cu") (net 9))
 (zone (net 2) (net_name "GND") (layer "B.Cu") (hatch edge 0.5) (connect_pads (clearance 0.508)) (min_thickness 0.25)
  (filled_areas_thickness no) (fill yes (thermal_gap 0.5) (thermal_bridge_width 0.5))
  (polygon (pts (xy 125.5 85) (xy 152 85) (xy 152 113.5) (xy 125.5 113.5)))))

